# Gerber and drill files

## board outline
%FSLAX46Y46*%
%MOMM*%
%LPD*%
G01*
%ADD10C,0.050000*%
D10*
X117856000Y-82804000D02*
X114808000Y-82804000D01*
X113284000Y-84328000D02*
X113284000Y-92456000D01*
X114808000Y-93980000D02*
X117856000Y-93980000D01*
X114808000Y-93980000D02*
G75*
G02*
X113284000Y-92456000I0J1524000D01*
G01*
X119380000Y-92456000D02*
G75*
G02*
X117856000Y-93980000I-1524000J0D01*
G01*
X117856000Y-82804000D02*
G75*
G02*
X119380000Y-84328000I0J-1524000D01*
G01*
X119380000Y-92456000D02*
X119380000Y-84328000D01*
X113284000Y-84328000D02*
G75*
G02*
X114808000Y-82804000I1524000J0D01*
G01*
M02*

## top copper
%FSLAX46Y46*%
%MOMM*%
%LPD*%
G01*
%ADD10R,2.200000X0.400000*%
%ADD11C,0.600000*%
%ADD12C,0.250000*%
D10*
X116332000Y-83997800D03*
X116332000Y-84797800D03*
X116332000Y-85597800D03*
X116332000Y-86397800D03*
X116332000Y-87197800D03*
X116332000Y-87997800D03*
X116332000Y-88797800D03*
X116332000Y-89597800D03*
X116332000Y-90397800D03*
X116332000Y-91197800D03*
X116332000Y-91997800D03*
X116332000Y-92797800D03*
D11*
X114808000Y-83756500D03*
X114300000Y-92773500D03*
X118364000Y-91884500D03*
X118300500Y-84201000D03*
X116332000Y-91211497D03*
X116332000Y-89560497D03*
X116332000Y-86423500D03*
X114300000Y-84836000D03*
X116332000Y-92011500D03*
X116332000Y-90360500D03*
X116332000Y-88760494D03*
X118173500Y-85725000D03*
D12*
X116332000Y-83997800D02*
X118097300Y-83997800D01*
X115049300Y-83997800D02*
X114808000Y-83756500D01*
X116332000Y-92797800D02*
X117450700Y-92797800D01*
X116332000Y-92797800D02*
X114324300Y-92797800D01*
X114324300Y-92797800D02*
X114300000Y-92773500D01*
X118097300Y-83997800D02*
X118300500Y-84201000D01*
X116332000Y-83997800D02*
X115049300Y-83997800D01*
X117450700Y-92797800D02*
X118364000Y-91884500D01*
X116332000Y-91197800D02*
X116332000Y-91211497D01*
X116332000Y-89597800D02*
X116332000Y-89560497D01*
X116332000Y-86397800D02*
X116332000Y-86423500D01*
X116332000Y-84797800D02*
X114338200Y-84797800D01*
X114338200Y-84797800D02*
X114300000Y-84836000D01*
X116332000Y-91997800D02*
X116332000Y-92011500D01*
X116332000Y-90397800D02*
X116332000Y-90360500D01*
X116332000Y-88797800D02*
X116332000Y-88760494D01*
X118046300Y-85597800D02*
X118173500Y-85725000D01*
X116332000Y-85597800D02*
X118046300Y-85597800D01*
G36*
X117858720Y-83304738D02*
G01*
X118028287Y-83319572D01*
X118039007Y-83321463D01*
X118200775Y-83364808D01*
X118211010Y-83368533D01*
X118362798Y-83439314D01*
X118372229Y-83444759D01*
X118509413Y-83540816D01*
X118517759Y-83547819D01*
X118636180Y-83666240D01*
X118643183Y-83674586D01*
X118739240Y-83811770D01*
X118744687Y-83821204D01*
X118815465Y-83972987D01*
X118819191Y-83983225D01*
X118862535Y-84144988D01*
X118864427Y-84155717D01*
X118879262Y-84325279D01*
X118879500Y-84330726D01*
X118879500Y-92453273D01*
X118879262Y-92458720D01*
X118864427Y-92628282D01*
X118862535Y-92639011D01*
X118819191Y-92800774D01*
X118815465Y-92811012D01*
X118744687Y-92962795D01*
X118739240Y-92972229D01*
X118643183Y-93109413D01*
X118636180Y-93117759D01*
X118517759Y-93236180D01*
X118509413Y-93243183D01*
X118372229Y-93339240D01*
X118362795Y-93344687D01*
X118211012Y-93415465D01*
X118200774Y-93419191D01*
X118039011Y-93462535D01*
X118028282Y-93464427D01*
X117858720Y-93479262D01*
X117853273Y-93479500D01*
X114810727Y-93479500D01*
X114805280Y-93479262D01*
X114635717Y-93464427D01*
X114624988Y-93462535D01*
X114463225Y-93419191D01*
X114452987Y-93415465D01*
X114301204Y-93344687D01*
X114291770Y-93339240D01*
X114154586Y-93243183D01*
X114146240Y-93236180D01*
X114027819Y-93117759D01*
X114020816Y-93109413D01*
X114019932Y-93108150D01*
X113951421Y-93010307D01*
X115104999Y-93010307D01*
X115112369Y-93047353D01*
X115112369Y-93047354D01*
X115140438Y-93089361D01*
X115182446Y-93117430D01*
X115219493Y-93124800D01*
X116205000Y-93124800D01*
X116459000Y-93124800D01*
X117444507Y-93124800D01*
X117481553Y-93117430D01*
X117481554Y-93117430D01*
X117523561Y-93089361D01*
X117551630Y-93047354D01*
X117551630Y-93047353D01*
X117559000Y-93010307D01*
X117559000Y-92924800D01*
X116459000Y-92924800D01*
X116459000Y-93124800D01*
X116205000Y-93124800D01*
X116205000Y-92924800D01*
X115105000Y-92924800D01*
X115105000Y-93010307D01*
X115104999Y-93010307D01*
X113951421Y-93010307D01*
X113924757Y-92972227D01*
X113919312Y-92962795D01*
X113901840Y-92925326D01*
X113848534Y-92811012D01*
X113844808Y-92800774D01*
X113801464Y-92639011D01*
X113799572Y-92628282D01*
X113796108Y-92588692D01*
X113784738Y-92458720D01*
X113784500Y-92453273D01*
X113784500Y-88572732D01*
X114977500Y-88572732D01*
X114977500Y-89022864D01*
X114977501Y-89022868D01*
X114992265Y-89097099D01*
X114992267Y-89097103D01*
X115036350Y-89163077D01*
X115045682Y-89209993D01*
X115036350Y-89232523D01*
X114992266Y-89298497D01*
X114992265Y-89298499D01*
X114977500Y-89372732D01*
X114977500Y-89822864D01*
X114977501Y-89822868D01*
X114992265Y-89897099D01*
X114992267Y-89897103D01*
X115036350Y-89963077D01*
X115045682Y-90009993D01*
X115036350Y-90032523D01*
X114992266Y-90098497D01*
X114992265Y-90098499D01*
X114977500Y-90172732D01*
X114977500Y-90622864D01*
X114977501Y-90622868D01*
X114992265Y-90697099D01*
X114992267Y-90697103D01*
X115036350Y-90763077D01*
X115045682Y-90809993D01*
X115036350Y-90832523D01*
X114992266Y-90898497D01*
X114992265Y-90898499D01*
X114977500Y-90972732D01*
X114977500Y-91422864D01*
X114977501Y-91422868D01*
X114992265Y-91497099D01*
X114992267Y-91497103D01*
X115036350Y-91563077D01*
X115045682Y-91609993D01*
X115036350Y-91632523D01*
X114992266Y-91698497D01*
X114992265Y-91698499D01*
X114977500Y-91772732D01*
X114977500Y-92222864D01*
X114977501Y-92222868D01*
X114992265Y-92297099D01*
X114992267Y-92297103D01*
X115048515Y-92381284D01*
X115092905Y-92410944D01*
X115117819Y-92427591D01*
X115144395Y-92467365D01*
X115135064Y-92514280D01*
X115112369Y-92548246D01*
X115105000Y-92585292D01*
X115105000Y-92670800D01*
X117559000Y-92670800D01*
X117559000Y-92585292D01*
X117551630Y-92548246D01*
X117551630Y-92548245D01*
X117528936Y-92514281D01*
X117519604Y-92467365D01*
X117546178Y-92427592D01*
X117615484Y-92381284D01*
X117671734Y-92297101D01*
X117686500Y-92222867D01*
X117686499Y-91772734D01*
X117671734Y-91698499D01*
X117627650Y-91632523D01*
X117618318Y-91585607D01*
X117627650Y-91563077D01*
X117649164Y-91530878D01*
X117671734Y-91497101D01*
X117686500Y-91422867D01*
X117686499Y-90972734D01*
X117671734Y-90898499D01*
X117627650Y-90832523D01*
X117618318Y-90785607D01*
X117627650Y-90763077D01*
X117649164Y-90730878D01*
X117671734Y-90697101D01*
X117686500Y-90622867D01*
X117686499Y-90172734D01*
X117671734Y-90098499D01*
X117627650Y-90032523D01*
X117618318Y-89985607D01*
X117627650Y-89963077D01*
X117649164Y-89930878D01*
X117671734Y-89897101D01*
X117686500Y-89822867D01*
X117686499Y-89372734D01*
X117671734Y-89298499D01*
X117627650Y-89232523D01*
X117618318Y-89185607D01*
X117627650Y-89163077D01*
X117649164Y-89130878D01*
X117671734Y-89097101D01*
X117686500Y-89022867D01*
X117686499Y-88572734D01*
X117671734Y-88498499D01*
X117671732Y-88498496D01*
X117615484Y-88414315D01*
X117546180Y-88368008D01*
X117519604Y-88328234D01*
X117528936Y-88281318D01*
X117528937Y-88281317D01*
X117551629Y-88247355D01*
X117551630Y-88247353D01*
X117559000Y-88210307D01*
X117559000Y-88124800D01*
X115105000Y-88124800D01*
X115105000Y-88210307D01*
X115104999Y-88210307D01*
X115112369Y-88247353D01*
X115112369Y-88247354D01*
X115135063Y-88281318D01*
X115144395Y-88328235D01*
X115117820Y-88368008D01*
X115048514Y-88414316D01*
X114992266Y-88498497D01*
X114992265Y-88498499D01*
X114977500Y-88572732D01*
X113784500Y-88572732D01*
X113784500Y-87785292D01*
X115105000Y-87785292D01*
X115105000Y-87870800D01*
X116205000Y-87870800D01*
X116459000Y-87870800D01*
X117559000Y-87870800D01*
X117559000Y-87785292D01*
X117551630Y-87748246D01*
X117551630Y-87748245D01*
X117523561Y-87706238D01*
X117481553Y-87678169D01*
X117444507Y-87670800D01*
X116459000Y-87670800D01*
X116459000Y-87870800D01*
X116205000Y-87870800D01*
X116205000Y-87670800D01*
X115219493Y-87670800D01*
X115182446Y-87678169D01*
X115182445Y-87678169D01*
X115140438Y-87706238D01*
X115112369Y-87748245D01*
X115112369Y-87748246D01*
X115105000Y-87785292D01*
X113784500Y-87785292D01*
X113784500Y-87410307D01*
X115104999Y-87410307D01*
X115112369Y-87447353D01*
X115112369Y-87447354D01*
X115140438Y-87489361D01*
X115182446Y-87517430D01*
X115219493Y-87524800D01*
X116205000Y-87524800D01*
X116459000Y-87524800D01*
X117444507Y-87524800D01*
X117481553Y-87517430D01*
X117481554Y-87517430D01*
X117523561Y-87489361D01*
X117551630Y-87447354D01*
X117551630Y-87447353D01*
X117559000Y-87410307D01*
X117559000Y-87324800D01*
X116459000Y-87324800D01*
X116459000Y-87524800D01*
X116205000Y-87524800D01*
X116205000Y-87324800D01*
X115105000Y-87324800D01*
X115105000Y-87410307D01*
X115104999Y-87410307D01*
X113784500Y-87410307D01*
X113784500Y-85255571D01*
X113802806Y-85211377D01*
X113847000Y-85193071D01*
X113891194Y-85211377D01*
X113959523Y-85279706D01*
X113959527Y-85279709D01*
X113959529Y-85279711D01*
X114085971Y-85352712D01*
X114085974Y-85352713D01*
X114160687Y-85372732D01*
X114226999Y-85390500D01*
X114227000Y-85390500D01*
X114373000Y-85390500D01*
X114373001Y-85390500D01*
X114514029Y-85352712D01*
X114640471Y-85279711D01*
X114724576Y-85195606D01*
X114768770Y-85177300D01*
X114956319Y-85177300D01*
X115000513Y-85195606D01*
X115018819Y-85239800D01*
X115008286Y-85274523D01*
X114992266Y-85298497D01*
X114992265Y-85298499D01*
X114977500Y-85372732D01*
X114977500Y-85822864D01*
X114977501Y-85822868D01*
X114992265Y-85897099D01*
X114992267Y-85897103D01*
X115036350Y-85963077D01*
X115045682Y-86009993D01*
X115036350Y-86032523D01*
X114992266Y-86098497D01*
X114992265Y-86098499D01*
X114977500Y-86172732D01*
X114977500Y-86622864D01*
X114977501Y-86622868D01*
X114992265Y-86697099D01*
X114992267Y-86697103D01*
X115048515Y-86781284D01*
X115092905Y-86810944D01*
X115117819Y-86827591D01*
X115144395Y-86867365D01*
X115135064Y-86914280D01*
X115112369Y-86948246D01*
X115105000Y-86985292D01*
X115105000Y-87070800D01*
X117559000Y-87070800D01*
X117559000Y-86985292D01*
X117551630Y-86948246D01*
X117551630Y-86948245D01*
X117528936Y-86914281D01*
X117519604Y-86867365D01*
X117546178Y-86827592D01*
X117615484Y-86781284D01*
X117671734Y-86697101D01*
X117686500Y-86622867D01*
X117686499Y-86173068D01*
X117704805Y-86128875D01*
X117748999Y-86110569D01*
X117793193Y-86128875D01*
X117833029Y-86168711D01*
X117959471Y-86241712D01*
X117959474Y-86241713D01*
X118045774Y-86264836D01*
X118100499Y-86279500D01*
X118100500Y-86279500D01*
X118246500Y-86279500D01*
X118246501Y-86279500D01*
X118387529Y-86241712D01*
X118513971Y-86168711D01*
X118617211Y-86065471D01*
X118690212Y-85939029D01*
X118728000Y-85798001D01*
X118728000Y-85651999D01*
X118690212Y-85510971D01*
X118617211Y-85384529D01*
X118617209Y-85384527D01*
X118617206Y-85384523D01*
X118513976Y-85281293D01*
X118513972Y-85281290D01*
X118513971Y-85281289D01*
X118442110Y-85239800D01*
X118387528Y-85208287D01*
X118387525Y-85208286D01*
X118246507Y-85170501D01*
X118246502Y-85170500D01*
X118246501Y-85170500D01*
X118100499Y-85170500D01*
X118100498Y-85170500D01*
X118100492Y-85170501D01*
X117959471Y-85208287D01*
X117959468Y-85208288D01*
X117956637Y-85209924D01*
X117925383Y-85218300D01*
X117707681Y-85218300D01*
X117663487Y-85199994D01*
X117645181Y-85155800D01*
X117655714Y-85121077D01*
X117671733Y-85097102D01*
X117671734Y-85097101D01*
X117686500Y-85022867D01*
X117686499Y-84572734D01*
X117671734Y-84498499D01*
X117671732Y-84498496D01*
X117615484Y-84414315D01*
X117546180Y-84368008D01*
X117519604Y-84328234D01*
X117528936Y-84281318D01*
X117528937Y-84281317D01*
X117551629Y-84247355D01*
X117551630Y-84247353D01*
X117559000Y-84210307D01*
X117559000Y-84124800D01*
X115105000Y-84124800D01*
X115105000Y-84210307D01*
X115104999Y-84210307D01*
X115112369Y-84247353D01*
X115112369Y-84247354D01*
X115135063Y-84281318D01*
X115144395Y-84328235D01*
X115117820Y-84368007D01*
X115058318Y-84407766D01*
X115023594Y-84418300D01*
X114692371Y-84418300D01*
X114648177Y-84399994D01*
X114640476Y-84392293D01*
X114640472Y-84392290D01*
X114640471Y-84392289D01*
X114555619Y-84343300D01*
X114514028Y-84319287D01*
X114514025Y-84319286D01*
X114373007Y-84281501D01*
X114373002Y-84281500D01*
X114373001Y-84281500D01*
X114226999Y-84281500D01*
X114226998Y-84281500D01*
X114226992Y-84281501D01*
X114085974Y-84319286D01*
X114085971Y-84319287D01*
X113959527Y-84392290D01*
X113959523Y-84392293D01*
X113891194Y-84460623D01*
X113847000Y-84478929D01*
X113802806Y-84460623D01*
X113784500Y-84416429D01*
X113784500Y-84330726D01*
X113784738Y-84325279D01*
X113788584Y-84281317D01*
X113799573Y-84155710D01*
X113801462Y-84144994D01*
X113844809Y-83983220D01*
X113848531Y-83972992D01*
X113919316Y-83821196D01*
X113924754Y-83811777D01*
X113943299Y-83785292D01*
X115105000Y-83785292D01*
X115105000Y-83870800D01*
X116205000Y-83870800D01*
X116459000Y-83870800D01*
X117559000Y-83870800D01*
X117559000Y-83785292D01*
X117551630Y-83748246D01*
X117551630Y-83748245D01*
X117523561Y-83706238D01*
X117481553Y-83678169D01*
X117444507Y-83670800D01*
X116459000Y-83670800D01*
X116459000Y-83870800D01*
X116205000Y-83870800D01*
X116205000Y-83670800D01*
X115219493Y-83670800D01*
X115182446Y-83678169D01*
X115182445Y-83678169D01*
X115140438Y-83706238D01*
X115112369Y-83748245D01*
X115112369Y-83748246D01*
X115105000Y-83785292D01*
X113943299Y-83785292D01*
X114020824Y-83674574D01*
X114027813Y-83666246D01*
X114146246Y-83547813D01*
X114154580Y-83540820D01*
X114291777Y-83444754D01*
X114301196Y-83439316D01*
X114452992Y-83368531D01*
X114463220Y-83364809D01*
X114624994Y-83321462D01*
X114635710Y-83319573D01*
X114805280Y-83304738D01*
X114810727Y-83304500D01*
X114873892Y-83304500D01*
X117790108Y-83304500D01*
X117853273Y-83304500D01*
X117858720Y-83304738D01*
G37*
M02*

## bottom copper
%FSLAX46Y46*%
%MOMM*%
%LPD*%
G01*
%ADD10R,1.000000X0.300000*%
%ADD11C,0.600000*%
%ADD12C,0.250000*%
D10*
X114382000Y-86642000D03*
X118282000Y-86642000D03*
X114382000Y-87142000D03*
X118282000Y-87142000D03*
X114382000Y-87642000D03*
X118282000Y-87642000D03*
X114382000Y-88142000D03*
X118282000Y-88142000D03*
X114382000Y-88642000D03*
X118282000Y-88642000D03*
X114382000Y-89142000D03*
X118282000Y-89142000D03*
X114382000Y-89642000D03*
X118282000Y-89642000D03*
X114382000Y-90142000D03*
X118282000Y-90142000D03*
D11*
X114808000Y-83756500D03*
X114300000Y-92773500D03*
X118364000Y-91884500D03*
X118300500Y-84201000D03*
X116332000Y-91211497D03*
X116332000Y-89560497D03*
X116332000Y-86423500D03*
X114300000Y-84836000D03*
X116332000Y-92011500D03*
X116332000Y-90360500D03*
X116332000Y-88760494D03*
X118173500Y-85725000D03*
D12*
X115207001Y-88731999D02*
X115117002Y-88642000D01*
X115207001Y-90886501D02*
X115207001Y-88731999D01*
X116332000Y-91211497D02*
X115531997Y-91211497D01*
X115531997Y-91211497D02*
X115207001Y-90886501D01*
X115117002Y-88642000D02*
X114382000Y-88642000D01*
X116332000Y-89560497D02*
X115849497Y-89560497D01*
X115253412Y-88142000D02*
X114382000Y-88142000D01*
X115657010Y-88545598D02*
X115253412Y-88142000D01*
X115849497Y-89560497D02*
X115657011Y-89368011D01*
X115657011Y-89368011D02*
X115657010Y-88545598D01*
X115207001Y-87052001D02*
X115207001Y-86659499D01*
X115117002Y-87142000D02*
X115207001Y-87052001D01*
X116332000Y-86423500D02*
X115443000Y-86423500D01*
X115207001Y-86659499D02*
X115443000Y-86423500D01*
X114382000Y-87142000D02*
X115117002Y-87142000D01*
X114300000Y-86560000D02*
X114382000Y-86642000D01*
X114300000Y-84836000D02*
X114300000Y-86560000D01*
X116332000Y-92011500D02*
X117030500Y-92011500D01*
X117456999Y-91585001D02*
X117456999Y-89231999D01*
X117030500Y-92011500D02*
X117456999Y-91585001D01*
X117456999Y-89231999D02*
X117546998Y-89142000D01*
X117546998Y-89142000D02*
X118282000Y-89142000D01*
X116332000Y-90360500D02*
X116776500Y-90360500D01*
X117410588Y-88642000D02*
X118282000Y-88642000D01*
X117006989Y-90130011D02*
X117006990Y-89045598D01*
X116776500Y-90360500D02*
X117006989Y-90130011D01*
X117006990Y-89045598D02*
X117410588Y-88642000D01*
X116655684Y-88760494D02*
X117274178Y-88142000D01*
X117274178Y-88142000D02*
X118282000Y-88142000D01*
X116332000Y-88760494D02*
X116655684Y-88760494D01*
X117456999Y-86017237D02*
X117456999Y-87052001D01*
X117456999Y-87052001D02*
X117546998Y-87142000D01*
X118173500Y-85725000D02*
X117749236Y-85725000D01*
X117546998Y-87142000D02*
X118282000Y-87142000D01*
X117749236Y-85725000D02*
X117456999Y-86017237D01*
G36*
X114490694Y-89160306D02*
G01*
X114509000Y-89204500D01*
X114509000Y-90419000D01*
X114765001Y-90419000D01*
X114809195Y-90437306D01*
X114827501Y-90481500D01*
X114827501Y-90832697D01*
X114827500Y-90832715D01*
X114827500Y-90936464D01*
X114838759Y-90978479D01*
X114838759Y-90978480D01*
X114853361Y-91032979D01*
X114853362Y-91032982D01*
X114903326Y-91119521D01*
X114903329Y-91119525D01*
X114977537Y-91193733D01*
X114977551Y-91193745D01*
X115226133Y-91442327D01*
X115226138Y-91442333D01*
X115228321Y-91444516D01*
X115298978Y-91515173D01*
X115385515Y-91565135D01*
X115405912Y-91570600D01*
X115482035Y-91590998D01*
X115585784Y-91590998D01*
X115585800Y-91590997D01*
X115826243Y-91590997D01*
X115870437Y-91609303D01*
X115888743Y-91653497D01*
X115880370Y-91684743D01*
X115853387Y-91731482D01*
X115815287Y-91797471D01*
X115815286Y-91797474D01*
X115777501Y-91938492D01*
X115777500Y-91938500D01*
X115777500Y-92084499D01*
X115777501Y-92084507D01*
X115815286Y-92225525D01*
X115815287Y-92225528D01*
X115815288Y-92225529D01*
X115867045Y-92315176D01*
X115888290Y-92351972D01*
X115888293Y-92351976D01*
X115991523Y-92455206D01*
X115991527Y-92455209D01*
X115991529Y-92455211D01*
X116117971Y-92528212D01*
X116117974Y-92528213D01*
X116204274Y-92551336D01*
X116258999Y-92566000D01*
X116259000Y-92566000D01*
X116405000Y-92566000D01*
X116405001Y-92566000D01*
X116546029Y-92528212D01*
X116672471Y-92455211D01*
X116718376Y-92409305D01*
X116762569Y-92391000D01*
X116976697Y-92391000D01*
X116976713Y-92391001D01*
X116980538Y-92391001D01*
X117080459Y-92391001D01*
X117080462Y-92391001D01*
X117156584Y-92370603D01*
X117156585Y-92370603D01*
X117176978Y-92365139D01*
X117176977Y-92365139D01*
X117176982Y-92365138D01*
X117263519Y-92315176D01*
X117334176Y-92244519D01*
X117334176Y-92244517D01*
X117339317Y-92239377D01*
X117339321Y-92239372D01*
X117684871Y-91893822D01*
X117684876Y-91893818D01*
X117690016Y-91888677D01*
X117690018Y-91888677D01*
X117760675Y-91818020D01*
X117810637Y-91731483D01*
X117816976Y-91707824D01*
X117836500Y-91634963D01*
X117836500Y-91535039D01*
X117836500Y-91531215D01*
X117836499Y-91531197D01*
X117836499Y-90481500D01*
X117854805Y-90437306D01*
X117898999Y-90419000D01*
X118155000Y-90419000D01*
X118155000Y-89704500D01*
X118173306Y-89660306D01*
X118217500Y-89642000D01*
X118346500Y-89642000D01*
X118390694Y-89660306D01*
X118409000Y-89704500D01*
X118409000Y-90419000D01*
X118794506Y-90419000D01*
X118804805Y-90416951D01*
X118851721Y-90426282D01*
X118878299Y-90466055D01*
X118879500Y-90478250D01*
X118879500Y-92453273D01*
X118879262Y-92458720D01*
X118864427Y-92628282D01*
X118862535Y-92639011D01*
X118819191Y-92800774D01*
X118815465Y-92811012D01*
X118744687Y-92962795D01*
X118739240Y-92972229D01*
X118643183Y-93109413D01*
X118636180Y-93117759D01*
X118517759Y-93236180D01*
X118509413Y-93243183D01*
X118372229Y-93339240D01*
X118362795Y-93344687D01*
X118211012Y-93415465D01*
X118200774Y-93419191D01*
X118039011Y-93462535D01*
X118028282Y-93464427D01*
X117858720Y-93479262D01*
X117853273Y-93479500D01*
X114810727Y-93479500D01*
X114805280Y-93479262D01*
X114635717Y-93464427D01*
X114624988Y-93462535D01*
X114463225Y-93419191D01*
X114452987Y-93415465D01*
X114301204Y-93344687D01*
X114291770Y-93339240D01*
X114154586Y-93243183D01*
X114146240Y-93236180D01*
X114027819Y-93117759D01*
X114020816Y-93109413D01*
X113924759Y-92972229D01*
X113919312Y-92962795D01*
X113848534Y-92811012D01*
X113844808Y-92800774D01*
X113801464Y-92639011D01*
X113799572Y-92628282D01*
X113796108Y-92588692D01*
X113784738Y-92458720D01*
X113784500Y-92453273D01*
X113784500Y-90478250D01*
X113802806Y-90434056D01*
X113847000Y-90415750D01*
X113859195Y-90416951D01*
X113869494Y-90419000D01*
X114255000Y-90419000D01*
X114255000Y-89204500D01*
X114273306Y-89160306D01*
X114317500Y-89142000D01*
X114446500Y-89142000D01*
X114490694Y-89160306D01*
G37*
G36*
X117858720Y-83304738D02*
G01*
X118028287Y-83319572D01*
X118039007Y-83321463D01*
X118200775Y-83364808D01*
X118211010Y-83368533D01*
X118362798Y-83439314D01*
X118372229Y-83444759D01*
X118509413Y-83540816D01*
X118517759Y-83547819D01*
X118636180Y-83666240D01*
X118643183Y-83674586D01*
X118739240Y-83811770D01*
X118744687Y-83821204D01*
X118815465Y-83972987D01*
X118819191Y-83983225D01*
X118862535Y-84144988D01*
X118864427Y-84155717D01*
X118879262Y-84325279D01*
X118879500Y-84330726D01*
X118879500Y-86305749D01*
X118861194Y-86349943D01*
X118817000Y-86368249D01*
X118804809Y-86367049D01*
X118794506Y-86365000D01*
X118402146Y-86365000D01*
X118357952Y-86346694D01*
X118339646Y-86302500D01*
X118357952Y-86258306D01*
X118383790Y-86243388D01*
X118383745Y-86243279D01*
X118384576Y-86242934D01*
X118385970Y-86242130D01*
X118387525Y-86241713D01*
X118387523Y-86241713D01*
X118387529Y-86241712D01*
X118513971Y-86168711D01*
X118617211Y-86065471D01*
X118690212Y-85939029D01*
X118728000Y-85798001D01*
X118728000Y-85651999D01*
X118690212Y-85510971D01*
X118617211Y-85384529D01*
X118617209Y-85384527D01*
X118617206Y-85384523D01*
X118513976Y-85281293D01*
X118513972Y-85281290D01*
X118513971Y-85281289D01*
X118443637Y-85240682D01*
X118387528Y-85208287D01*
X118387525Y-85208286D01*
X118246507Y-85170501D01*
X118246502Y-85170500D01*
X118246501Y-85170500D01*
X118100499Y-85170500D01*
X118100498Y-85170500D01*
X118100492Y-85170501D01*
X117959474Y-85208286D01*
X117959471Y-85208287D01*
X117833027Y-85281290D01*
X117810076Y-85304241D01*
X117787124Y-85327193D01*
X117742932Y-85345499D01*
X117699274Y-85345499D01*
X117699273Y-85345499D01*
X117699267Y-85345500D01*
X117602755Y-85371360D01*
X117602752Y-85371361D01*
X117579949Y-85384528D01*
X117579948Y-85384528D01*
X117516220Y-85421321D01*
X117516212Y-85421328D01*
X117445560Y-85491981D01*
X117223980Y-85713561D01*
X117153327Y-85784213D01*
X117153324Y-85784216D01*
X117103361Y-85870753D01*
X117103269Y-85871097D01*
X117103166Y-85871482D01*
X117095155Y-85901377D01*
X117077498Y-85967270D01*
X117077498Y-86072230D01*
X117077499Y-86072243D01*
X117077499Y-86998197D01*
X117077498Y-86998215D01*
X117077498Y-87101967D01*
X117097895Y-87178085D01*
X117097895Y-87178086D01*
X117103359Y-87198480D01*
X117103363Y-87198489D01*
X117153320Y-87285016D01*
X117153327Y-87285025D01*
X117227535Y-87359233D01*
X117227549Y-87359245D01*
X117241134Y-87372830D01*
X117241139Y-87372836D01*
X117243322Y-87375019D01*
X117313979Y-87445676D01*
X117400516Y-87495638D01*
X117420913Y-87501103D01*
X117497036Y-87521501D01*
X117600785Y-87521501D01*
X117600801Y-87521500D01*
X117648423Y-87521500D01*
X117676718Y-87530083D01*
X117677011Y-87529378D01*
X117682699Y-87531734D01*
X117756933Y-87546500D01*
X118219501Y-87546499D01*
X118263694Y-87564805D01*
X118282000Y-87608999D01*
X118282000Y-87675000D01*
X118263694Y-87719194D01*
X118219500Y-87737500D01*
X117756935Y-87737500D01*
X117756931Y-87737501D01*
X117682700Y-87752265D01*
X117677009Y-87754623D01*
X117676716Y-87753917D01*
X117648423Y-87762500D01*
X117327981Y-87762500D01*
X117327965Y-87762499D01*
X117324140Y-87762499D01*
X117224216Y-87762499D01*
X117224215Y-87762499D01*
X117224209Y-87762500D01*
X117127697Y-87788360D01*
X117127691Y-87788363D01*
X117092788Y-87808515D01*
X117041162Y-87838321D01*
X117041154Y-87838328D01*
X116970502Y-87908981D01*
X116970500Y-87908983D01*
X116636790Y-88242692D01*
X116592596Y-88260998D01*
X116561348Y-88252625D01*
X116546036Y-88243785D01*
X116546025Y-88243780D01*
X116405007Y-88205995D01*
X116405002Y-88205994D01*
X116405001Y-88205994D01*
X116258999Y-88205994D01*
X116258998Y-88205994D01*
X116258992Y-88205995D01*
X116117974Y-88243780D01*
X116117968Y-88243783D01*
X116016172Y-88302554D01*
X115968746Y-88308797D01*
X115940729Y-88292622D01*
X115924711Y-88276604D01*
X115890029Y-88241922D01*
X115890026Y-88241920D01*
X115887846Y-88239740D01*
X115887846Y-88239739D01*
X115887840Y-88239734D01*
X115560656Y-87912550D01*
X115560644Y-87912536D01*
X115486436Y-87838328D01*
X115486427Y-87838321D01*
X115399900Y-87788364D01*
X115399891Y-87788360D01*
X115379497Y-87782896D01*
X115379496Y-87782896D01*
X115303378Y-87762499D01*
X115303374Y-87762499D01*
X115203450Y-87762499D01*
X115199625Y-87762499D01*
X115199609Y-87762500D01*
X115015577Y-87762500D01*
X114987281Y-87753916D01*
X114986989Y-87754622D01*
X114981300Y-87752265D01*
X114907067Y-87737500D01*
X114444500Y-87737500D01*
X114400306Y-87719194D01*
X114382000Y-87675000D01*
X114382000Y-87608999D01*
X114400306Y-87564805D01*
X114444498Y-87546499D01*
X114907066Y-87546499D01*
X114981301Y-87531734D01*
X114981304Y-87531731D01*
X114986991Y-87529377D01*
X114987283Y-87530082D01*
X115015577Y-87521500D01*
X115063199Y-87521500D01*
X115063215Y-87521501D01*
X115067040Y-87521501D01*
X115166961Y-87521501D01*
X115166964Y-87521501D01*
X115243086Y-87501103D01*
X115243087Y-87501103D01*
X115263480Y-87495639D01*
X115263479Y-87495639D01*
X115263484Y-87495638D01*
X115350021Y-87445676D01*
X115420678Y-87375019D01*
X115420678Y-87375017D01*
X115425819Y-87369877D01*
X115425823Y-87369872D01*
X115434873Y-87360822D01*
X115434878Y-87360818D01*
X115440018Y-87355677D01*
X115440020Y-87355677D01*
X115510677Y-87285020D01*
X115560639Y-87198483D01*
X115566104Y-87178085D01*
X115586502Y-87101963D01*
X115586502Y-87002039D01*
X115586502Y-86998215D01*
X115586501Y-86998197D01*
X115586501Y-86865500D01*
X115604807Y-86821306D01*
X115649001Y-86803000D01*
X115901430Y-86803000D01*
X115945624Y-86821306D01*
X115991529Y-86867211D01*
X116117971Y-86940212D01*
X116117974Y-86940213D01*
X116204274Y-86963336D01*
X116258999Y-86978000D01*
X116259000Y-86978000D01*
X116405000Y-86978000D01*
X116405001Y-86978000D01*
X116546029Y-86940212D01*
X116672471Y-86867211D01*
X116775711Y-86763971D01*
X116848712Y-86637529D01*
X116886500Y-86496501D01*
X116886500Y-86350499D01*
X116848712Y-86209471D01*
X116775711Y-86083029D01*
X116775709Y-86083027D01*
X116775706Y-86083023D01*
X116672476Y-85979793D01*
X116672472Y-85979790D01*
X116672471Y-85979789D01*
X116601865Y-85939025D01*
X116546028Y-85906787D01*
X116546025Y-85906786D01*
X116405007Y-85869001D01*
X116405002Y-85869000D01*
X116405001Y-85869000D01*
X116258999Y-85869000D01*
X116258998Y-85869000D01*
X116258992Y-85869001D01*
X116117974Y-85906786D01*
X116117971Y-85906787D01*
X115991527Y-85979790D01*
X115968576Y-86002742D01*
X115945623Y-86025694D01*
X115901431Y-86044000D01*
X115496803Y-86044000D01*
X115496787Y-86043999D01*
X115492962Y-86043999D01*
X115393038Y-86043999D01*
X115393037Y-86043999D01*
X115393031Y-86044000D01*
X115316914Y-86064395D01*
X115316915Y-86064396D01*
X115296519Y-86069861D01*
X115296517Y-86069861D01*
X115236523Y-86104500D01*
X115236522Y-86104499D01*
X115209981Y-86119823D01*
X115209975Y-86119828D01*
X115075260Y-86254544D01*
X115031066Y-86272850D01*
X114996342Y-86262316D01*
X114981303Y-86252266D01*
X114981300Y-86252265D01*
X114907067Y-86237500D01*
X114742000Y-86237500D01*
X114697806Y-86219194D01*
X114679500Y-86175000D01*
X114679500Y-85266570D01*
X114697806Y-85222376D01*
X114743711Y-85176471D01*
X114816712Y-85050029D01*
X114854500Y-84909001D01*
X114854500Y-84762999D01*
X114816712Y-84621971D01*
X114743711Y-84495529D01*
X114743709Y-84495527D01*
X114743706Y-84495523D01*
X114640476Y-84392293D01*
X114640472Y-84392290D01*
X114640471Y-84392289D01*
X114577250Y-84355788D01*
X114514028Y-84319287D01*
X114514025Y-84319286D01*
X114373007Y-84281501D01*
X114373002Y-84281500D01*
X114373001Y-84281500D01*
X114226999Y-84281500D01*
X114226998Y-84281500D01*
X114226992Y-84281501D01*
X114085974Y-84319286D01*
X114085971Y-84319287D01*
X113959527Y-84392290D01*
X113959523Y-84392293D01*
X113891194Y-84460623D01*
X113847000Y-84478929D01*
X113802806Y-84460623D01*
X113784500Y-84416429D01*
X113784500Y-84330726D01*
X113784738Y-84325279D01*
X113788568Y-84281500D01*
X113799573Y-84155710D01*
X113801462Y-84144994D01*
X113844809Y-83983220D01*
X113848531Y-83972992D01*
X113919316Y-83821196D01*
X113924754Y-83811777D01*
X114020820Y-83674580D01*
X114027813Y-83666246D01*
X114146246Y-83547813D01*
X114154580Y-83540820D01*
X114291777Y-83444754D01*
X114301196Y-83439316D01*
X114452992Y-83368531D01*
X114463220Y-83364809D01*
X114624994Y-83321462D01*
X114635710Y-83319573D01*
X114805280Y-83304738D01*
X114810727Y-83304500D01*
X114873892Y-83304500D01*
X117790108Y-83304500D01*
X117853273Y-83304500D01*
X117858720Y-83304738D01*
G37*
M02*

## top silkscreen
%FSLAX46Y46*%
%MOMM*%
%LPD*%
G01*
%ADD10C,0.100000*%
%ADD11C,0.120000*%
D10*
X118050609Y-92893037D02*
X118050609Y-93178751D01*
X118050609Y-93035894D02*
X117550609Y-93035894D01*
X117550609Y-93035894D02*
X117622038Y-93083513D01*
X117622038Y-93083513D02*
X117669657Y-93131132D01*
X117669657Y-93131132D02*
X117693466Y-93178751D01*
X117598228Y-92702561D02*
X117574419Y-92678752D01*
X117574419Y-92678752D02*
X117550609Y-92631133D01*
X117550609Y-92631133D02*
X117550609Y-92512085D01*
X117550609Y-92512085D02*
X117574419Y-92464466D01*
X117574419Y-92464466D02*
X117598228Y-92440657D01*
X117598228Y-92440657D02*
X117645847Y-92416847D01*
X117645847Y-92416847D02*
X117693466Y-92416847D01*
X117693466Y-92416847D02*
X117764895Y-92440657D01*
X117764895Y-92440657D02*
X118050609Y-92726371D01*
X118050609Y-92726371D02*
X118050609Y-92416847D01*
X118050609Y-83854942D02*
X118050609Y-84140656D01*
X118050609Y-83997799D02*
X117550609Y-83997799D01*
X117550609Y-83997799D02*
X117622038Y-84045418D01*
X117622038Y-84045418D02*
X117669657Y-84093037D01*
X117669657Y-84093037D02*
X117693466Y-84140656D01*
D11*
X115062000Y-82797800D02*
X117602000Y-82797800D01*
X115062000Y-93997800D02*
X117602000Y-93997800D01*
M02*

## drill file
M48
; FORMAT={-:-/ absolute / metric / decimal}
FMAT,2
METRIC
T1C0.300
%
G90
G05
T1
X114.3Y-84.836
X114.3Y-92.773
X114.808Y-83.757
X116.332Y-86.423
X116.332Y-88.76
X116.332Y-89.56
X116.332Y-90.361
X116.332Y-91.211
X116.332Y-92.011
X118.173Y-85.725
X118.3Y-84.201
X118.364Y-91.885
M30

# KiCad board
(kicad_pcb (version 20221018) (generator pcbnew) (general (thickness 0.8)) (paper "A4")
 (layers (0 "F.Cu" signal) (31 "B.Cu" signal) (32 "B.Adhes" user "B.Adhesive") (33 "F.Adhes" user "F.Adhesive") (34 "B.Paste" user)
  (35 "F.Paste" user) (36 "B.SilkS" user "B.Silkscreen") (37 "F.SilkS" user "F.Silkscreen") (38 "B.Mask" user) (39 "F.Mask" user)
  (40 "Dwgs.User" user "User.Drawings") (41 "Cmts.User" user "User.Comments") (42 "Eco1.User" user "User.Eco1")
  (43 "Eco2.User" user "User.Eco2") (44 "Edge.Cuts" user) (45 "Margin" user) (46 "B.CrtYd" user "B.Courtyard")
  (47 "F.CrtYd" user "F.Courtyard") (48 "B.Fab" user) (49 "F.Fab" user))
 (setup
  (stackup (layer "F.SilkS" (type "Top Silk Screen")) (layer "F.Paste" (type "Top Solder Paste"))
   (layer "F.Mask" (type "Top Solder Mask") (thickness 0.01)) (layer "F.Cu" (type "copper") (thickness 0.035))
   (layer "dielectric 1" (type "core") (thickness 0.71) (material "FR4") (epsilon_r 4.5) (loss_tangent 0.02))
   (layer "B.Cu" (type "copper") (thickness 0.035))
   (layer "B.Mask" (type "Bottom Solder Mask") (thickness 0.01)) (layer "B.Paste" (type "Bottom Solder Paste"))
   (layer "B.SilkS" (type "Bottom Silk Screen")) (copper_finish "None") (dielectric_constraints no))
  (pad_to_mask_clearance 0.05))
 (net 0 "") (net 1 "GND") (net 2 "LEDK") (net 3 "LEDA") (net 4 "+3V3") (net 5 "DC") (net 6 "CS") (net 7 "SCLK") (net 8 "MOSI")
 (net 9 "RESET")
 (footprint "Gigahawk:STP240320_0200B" (layer "F.Cu") (at 116.332 83.9978)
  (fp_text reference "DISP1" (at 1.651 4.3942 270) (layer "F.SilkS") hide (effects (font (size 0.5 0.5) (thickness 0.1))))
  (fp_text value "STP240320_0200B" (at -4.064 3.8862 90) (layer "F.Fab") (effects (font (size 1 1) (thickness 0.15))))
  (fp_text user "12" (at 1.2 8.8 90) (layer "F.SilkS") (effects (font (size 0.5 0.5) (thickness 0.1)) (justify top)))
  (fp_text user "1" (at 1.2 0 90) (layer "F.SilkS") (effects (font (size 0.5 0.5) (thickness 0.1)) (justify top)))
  (fp_line (start -1.27 -1.2) (end 1.27 -1.2) (stroke (width 0.12) (type solid)) (layer "F.SilkS"))
  (fp_line (start -1.27 10) (end 1.27 10) (stroke (width 0.12) (type solid)) (layer "F.SilkS"))
  (pad "1" smd rect (at 0 0 90) (size 0.4 2.2) (layers "F.Cu" "F.Paste" "F.Mask") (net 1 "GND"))
  (pad "2" smd rect (at 0 0.8 90) (size 0.4 2.2) (layers "F.Cu" "F.Paste" "F.Mask") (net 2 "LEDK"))
  (pad "3" smd rect (at 0 1.6 90) (size 0.4 2.2) (layers "F.Cu" "F.Paste" "F.Mask") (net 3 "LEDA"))
  (pad "4" smd rect (at 0 2.4 90) (size 0.4 2.2) (layers "F.Cu" "F.Paste" "F.Mask") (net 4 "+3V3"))
  (pad "5" smd rect (at 0 3.2 90) (size 0.4 2.2) (layers "F.Cu" "F.Paste" "F.Mask") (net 1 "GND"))
  (pad "6" smd rect (at 0 4 90) (size 0.4 2.2) (layers "F.Cu" "F.Paste" "F.Mask") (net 1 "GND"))
  (pad "7" smd rect (at 0 4.8 90) (size 0.4 2.2) (layers "F.Cu" "F.Paste" "F.Mask") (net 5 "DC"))
  (pad "8" smd rect (at 0 5.6 90) (size 0.4 2.2) (layers "F.Cu" "F.Paste" "F.Mask") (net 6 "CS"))
  (pad "9" smd rect (at 0 6.4 90) (size 0.4 2.2) (layers "F.Cu" "F.Paste" "F.Mask") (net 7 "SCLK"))
  (pad "10" smd rect (at 0 7.2 90) (size 0.4 2.2) (layers "F.Cu" "F.Paste" "F.Mask") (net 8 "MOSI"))
  (pad "11" smd rect (at 0 8 90) (size 0.4 2.2) (layers "F.Cu" "F.Paste" "F.Mask") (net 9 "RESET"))
  (pad "12" smd rect (at 0 8.8 90) (size 0.4 2.2) (layers "F.Cu" "F.Paste" "F.Mask") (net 1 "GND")))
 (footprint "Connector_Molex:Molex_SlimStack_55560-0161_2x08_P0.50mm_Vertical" (layer "B.Cu") (at 116.332 88.392 -90)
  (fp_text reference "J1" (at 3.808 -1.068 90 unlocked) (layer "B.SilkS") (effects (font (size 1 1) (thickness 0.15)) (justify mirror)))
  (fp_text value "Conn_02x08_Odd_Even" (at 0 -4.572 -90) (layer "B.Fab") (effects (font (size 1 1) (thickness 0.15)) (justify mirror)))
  (pad "1" smd rect (at -1.75 1.95 270) (size 0.3 1) (layers "B.Cu" "B.Paste" "B.Mask") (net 2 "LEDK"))
  (pad "2" smd rect (at -1.75 -1.95 270) (size 0.3 1) (layers "B.Cu" "B.Paste" "B.Mask") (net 1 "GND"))
  (pad "3" smd rect (at -1.25 1.95 270) (size 0.3 1) (layers "B.Cu" "B.Paste" "B.Mask") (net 4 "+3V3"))
  (pad "4" smd rect (at -1.25 -1.95 270) (size 0.3 1) (layers "B.Cu" "B.Paste" "B.Mask") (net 3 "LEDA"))
  (pad "5" smd rect (at -0.75 1.95 270) (size 0.3 1) (layers "B.Cu" "B.Paste" "B.Mask") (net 1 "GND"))
  (pad "6" smd rect (at -0.75 -1.95 270) (size 0.3 1) (layers "B.Cu" "B.Paste" "B.Mask") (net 1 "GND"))
  (pad "7" smd rect (at -0.25 1.95 270) (size 0.3 1) (layers "B.Cu" "B.Paste" "B.Mask") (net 6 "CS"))
  (pad "8" smd rect (at -0.25 -1.95 270) (size 0.3 1) (layers "B.Cu" "B.Paste" "B.Mask") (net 5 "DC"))
  (pad "9" smd rect (at 0.25 1.95 270) (size 0.3 1) (layers "B.Cu" "B.Paste" "B.Mask") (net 8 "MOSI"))
  (pad "10" smd rect (at 0.25 -1.95 270) (size 0.3 1) (layers "B.Cu" "B.Paste" "B.Mask") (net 7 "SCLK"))
  (pad "11" smd rect (at 0.75 1.95 270) (size 0.3 1) (layers "B.Cu" "B.Paste" "B.Mask") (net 1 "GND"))
  (pad "12" smd rect (at 0.75 -1.95 270) (size 0.3 1) (layers "B.Cu" "B.Paste" "B.Mask") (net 9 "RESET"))
  (pad "13" smd rect (at 1.25 1.95 270) (size 0.3 1) (layers "B.Cu" "B.Paste" "B.Mask") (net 1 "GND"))
  (pad "14" smd rect (at 1.25 -1.95 270) (size 0.3 1) (layers "B.Cu" "B.Paste" "B.Mask") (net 1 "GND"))
  (pad "15" smd rect (at 1.75 1.95 270) (size 0.3 1) (layers "B.Cu" "B.Paste" "B.Mask") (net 1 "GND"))
  (pad "16" smd rect (at 1.75 -1.95 270) (size 0.3 1) (layers "B.Cu" "B.Paste" "B.Mask") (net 1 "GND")))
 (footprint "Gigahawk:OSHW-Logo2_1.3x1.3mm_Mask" (layer "B.Cu") (at 116.4 84.2 -90)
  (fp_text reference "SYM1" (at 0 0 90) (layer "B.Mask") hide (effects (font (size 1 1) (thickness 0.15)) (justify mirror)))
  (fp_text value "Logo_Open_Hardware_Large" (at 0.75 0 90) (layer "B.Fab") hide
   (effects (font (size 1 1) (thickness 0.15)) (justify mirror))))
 (gr_line (start 117.856 82.804) (end 114.808 82.804) (stroke (width 0.05) (type solid)) (layer "Edge.Cuts"))
 (gr_line (start 113.284 84.328) (end 113.284 92.456) (stroke (width 0.05) (type solid)) (layer "Edge.Cuts"))
 (gr_line (start 114.808 93.98) (end 117.856 93.98) (stroke (width 0.05) (type solid)) (layer "Edge.Cuts"))
 (gr_arc (start 114.808 93.98) (mid 113.730369 93.533631) (end 113.284 92.456) (stroke (width 0.05) (type solid)) (layer "Edge.Cuts"))
 (gr_arc (start 119.38 92.456) (mid 118.933631 93.533631) (end 117.856 93.98) (stroke (width 0.05) (type solid)) (layer "Edge.Cuts"))
 (gr_arc (start 117.856 82.804) (mid 118.933631 83.250369) (end 119.38 84.328) (stroke (width 0.05) (type solid)) (layer "Edge.Cuts"))
 (gr_line (start 119.38 92.456) (end 119.38 84.328) (stroke (width 0.05) (type solid)) (layer "Edge.Cuts"))
 (gr_arc (start 113.284 84.328) (mid 113.730369 83.250369) (end 114.808 82.804) (stroke (width 0.05) (type solid)) (layer "Edge.Cuts"))
 (segment (start 116.332 83.9978) (end 118.0973 83.9978) (width 0.25) (layer "F.Cu") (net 1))
 (segment (start 115.0493 83.9978) (end 114.808 83.7565) (width 0.25) (layer "F.Cu") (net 1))
 (segment (start 116.332 92.7978) (end 117.4507 92.7978) (width 0.25) (layer "F.Cu") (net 1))
 (segment (start 116.332 92.7978) (end 114.3243 92.7978) (width 0.25) (layer "F.Cu") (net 1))
 (segment (start 114.3243 92.7978) (end 114.3 92.7735) (width 0.25) (layer "F.Cu") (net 1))
 (segment (start 118.0973 83.9978) (end 118.3005 84.201) (width 0.25) (layer "F.Cu") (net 1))
 (segment (start 116.332 83.9978) (end 115.0493 83.9978) (width 0.25) (layer "F.Cu") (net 1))
 (segment (start 117.4507 92.7978) (end 118.364 91.8845) (width 0.25) (layer "F.Cu") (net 1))
 (via (at 114.808 83.7565) (size 0.6) (drill 0.3) (layers "F.Cu" "B.Cu") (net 1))
 (via (at 114.3 92.7735) (size 0.6) (drill 0.3) (layers "F.Cu" "B.Cu") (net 1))
 (via (at 118.364 91.8845) (size 0.6) (drill 0.3) (layers "F.Cu" "B.Cu") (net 1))
 (via (at 118.3005 84.201) (size 0.6) (drill 0.3) (layers "F.Cu" "B.Cu") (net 1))
 (segment (start 116.332 91.1978) (end 116.332 91.211497) (width 0.25) (layer "F.Cu") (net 8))
 (via (at 116.332 91.211497) (size 0.6) (drill 0.3) (layers "F.Cu" "B.Cu") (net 8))
 (segment (start 115.207001 88.731999) (end 115.117002 88.642) (width 0.25) (layer "B.Cu") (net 8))
 (segment (start 115.207001 90.886501) (end 115.207001 88.731999) (width 0.25) (layer "B.Cu") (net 8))
 (segment (start 116.332 91.211497) (end 115.531997 91.211497) (width 0.25) (layer "B.Cu") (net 8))
 (segment (start 115.531997 91.211497) (end 115.207001 90.886501) (width 0.25) (layer "B.Cu") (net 8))
 (segment (start 115.117002 88.642) (end 114.382 88.642) (width 0.25) (layer "B.Cu") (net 8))
 (segment (start 116.332 89.5978) (end 116.332 89.560497) (width 0.25) (layer "F.Cu") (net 6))
 (via (at 116.332 89.560497) (size 0.6) (drill 0.3) (layers "F.Cu" "B.Cu") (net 6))
 (segment (start 116.332 89.560497) (end 115.849497 89.560497) (width 0.25) (layer "B.Cu") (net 6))
 (segment (start 115.253412 88.142) (end 114.382 88.142) (width 0.25) (layer "B.Cu") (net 6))
 (segment (start 115.65701 88.545598) (end 115.253412 88.142) (width 0.25) (layer "B.Cu") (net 6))
 (segment (start 115.849497 89.560497) (end 115.657011 89.368011) (width 0.25) (layer "B.Cu") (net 6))
 (segment (start 115.657011 89.368011) (end 115.65701 88.545598) (width 0.25) (layer "B.Cu") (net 6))
 (segment (start 116.332 86.3978) (end 116.332 86.4235) (width 0.25) (layer "F.Cu") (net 4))
 (via (at 116.332 86.4235) (size 0.6) (drill 0.3) (layers "F.Cu" "B.Cu") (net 4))
 (segment (start 115.207001 87.052001) (end 115.207001 86.659499) (width 0.25) (layer "B.Cu") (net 4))
 (segment (start 115.117002 87.142) (end 115.207001 87.052001) (width 0.25) (layer "B.Cu") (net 4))
 (segment (start 116.332 86.4235) (end 115.443 86.4235) (width 0.25) (layer "B.Cu") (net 4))
 (segment (start 115.207001 86.659499) (end 115.443 86.4235) (width 0.25) (layer "B.Cu") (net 4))
 (segment (start 114.382 87.142) (end 115.117002 87.142) (width 0.25) (layer "B.Cu") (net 4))
 (segment (start 116.332 84.7978) (end 114.3382 84.7978) (width 0.25) (layer "F.Cu") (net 2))
 (segment (start 114.3382 84.7978) (end 114.3 84.836) (width 0.25) (layer "F.Cu") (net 2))
 (via (at 114.3 84.836) (size 0.6) (drill 0.3) (layers "F.Cu" "B.Cu") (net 2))
 (segment (start 114.3 86.56) (end 114.382 86.642) (width 0.25) (layer "B.Cu") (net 2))
 (segment (start 114.3 84.836) (end 114.3 86.56) (width 0.25) (layer "B.Cu") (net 2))
 (segment (start 116.332 91.9978) (end 116.332 92.0115) (width 0.25) (layer "F.Cu") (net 9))
 (via (at 116.332 92.0115) (size 0.6) (drill 0.3) (layers "F.Cu" "B.Cu") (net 9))
 (segment (start 116.332 92.0115) (end 117.0305 92.0115) (width 0.25) (layer "B.Cu") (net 9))
 (segment (start 117.456999 91.585001) (end 117.456999 89.231999) (width 0.25) (layer "B.Cu") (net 9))
 (segment (start 117.0305 92.0115) (end 117.456999 91.585001) (width 0.25) (layer "B.Cu") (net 9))
 (segment (start 117.456999 89.231999) (end 117.546998 89.142) (width 0.25) (layer "B.Cu") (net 9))
 (segment (start 117.546998 89.142) (end 118.282 89.142) (width 0.25) (layer "B.Cu") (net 9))
 (segment (start 116.332 90.3978) (end 116.332 90.3605) (width 0.25) (layer "F.Cu") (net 7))
 (via (at 116.332 90.3605) (size 0.6) (drill 0.3) (layers "F.Cu" "B.Cu") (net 7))
 (segment (start 116.332 90.3605) (end 116.7765 90.3605) (width 0.25) (layer "B.Cu") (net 7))
 (segment (start 117.410588 88.642) (end 118.282 88.642) (width 0.25) (layer "B.Cu") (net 7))
 (segment (start 117.006989 90.130011) (end 117.00699 89.045598) (width 0.25) (layer "B.Cu") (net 7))
 (segment (start 116.7765 90.3605) (end 117.006989 90.130011) (width 0.25) (layer "B.Cu") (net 7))
 (segment (start 117.00699 89.045598) (end 117.410588 88.642) (width 0.25) (layer "B.Cu") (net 7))
 (segment (start 116.332 88.7978) (end 116.332 88.760494) (width 0.25) (layer "F.Cu") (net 5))
 (via (at 116.332 88.760494) (size 0.6) (drill 0.3) (layers "F.Cu" "B.Cu") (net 5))
 (segment (start 116.655684 88.760494) (end 117.274178 88.142) (width 0.25) (layer "B.Cu") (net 5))
 (segment (start 117.274178 88.142) (end 118.282 88.142) (width 0.25) (layer "B.Cu") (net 5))
 (segment (start 116.332 88.760494) (end 116.655684 88.760494) (width 0.25) (layer "B.Cu") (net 5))
 (segment (start 118.0463 85.5978) (end 118.1735 85.725) (width 0.25) (layer "F.Cu") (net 3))
 (segment (start 116.332 85.5978) (end 118.0463 85.5978) (width 0.25) (layer "F.Cu") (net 3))
 (via (at 118.1735 85.725) (size 0.6) (drill 0.3) (layers "F.Cu" "B.Cu") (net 3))
 (segment (start 117.456999 86.017237) (end 117.456999 87.052001) (width 0.25) (layer "B.Cu") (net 3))
 (segment (start 117.456999 87.052001) (end 117.546998 87.142) (width 0.25) (layer "B.Cu") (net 3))
 (segment (start 118.1735 85.725) (end 117.749236 85.725) (width 0.25) (layer "B.Cu") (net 3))
 (segment (start 117.546998 87.142) (end 118.282 87.142) (width 0.25) (layer "B.Cu") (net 3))
 (segment (start 117.749236 85.725) (end 117.456999 86.017237) (width 0.25) (layer "B.Cu") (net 3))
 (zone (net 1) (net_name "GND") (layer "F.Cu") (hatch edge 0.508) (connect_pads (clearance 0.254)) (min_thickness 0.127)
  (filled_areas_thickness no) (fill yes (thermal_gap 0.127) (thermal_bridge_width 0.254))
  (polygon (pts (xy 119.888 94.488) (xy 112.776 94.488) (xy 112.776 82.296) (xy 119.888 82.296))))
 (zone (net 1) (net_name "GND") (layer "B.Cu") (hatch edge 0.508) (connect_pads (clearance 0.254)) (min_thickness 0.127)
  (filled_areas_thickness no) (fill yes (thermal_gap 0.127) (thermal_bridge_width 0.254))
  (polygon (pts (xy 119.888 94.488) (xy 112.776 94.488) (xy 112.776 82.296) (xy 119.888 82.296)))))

